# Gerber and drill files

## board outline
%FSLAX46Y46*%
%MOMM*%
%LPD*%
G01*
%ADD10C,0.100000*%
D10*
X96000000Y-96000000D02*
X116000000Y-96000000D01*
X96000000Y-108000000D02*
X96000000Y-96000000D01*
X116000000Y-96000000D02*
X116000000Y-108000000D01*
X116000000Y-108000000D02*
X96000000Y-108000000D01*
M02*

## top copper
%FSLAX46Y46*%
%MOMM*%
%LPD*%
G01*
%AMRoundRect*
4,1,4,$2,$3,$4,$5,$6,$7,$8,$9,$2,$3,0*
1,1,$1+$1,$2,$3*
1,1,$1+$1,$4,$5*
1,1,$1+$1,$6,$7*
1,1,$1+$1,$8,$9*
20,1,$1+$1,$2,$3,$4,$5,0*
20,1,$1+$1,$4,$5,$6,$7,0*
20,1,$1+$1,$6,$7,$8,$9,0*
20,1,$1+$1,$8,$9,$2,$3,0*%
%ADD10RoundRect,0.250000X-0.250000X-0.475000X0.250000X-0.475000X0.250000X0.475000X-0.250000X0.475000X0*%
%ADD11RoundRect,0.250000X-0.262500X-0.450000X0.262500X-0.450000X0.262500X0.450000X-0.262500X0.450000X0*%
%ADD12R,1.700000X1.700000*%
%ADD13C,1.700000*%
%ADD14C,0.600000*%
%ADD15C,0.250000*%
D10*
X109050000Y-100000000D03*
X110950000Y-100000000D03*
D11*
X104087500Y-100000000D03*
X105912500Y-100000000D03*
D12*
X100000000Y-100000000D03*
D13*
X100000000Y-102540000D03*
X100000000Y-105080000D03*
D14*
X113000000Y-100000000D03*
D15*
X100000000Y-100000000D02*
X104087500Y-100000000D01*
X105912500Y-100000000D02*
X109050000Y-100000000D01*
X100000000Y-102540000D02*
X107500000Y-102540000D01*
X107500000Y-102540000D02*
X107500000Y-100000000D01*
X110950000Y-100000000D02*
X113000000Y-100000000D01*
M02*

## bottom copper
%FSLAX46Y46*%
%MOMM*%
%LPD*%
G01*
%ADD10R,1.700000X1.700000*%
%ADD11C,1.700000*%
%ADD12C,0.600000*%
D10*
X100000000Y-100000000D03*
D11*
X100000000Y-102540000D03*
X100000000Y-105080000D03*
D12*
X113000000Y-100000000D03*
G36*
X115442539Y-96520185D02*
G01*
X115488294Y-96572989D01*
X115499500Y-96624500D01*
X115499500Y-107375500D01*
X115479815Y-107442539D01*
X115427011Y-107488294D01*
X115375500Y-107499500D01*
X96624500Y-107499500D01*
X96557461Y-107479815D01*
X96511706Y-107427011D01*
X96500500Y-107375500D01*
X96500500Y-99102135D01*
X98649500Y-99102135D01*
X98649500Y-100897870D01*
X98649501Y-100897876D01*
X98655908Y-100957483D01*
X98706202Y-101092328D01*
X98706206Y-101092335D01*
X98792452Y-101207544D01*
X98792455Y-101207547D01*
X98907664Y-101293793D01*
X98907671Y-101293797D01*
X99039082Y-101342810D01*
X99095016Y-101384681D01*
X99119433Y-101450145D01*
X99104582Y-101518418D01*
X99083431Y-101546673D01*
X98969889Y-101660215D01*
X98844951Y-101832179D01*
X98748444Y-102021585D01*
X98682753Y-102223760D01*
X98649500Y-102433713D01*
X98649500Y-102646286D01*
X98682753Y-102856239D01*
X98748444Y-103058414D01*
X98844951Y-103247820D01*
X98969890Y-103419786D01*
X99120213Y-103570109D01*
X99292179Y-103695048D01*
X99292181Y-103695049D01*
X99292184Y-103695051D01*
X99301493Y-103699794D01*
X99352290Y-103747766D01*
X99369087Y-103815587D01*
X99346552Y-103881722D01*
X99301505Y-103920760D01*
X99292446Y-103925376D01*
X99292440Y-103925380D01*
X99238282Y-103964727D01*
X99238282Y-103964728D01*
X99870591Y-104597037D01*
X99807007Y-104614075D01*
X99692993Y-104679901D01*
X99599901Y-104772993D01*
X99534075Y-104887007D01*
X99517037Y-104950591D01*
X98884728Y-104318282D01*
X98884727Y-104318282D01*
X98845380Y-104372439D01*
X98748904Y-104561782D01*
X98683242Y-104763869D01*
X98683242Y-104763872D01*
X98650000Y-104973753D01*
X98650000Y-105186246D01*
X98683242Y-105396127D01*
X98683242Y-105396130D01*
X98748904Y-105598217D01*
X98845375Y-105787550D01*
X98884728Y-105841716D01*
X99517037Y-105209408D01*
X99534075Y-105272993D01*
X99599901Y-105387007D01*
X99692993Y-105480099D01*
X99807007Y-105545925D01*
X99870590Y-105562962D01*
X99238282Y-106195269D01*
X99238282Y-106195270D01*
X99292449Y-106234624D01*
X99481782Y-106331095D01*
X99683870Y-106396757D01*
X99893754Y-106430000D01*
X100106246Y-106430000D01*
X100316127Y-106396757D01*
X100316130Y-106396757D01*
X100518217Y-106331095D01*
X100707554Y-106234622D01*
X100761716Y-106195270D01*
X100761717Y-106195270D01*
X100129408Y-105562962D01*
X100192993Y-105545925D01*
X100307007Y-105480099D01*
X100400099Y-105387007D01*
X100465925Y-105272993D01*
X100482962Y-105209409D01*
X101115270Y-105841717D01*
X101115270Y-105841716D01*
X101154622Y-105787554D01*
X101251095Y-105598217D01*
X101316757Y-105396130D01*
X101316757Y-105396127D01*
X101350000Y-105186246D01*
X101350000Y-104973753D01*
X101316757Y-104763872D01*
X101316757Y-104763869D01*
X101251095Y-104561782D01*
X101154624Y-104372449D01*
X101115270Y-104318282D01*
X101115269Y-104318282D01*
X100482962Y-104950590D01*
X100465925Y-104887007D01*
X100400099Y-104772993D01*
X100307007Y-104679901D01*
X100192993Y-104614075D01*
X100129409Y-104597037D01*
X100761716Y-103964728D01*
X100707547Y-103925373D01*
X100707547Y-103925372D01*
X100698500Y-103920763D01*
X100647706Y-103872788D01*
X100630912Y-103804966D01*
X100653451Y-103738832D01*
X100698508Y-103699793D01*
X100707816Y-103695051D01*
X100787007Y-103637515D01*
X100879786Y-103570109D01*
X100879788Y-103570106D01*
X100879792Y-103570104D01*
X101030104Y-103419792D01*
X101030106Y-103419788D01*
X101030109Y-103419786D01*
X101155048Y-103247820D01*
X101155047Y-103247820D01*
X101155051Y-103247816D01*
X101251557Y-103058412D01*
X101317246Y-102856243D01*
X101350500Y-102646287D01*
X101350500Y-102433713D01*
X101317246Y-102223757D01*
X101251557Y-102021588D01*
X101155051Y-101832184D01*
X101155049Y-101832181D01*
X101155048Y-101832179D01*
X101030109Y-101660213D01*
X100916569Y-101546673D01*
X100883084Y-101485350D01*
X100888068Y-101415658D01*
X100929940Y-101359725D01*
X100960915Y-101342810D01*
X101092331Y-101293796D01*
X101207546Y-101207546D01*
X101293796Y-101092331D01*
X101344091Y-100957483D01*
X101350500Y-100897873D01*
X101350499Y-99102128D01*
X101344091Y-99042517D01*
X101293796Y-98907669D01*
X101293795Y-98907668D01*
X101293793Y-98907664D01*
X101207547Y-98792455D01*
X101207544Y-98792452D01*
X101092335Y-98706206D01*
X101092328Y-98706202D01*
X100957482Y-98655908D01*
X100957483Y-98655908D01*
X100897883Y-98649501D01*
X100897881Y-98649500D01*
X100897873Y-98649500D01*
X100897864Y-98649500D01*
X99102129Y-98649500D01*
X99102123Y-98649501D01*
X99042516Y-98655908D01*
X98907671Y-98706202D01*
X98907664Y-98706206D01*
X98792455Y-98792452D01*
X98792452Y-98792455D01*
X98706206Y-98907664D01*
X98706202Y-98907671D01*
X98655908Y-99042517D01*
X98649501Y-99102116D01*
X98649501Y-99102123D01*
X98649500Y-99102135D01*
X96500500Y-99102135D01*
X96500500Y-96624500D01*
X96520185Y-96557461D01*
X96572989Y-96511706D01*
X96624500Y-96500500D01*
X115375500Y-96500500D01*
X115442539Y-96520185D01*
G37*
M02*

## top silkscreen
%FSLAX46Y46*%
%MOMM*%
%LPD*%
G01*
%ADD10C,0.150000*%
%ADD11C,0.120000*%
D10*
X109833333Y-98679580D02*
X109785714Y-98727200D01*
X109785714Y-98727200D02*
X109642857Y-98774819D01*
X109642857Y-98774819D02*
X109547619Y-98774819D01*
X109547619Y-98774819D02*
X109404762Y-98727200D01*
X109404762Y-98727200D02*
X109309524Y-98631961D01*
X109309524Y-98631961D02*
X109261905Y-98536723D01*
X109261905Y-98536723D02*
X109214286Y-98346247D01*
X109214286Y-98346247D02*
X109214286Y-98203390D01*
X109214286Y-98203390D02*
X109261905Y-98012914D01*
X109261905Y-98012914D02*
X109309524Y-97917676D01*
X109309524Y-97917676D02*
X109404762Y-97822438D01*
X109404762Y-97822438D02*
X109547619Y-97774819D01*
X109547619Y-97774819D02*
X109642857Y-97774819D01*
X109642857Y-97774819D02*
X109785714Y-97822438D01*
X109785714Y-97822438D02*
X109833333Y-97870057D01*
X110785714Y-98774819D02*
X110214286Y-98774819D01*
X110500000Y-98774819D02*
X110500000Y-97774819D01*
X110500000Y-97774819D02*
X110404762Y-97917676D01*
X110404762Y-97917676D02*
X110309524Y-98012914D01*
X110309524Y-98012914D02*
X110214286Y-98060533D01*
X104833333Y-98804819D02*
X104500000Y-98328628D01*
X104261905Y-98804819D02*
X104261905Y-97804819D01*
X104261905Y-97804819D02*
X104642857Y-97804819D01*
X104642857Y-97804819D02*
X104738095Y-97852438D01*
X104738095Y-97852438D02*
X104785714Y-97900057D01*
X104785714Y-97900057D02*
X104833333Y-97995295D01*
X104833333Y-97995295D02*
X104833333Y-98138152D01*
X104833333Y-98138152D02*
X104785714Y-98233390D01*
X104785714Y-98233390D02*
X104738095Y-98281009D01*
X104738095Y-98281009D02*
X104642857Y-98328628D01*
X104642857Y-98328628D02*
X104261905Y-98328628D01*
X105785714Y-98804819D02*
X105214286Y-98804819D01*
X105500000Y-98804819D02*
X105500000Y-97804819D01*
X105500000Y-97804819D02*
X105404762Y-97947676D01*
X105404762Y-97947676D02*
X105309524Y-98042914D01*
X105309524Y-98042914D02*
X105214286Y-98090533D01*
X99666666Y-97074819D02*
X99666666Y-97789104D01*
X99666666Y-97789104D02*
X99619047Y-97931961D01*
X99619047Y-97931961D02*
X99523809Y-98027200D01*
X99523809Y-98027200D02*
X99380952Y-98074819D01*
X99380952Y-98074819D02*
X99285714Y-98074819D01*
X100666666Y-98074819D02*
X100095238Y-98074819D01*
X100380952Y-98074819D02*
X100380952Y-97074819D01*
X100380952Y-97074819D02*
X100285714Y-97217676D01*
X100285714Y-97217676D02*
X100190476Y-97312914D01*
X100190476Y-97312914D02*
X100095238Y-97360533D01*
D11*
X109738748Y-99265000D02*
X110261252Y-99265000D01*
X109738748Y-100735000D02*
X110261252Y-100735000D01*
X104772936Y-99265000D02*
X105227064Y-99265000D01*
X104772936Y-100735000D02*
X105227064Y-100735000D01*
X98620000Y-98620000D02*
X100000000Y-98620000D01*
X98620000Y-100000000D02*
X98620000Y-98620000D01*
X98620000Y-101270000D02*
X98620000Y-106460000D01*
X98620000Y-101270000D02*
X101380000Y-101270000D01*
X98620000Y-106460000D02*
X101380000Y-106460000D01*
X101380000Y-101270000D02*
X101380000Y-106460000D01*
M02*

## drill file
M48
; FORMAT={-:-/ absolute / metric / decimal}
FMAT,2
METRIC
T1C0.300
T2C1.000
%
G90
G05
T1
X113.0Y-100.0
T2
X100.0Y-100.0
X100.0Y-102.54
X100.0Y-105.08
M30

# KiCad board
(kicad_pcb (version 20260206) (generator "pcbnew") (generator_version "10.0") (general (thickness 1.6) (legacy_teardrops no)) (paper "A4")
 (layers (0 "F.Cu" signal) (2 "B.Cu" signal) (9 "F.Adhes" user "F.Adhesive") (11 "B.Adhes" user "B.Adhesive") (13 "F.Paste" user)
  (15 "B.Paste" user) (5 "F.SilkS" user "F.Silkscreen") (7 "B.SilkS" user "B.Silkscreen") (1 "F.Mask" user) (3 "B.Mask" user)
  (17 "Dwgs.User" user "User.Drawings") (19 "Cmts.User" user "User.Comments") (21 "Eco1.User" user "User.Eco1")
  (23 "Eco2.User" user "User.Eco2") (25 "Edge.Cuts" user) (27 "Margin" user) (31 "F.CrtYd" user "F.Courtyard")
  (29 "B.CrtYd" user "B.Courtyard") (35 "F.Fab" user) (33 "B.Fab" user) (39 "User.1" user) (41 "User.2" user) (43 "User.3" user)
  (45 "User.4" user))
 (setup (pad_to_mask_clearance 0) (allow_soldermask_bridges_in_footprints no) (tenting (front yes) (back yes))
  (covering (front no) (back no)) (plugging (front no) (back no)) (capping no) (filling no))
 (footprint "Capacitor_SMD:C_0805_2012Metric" (layer "F.Cu") (at 110 100)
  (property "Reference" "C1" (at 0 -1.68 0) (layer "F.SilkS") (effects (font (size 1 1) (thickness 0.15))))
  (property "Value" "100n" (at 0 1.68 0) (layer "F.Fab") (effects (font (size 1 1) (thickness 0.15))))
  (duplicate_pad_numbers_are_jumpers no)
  (fp_line (start -0.261252 -0.735) (end 0.261252 -0.735) (stroke (width 0.12) (type solid)) (layer "F.SilkS"))
  (fp_line (start -0.261252 0.735) (end 0.261252 0.735) (stroke (width 0.12) (type solid)) (layer "F.SilkS"))
  (pad "1" smd roundrect (at -0.95 0) (size 1 1.45) (layers "F.Cu" "F.Mask" "F.Paste") (roundrect_rratio 0.25) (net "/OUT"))
  (pad "2" smd roundrect (at 0.95 0) (size 1 1.45) (layers "F.Cu" "F.Mask" "F.Paste") (roundrect_rratio 0.25) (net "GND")))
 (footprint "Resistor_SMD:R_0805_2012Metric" (layer "F.Cu") (at 105 100)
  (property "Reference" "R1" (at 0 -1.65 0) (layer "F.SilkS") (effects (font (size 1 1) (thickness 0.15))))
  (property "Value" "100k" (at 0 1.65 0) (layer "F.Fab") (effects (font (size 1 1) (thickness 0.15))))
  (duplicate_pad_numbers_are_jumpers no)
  (fp_line (start -0.227064 -0.735) (end 0.227064 -0.735) (stroke (width 0.12) (type solid)) (layer "F.SilkS"))
  (fp_line (start -0.227064 0.735) (end 0.227064 0.735) (stroke (width 0.12) (type solid)) (layer "F.SilkS"))
  (pad "1" smd roundrect (at -0.9125 0) (size 1.025 1.4) (layers "F.Cu" "F.Mask" "F.Paste") (roundrect_rratio 0.243902) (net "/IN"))
  (pad "2" smd roundrect (at 0.9125 0) (size 1.025 1.4) (layers "F.Cu" "F.Mask" "F.Paste") (roundrect_rratio 0.243902) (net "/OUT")))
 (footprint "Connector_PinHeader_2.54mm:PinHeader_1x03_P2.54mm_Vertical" (layer "F.Cu") (at 100 100)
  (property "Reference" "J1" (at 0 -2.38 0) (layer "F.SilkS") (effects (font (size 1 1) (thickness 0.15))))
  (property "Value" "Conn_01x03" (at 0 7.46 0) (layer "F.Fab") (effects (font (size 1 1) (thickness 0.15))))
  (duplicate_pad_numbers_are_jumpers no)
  (fp_line (start -1.38 -1.38) (end 0 -1.38) (stroke (width 0.12) (type solid)) (layer "F.SilkS"))
  (fp_line (start -1.38 0) (end -1.38 -1.38) (stroke (width 0.12) (type solid)) (layer "F.SilkS"))
  (fp_line (start -1.38 1.27) (end -1.38 6.46) (stroke (width 0.12) (type solid)) (layer "F.SilkS"))
  (fp_line (start -1.38 1.27) (end 1.38 1.27) (stroke (width 0.12) (type solid)) (layer "F.SilkS"))
  (fp_line (start -1.38 6.46) (end 1.38 6.46) (stroke (width 0.12) (type solid)) (layer "F.SilkS"))
  (fp_line (start 1.38 1.27) (end 1.38 6.46) (stroke (width 0.12) (type solid)) (layer "F.SilkS"))
  (pad "1" thru_hole rect (at 0 0) (size 1.7 1.7) (drill 1) (layers "*.Cu" "*.Mask") (remove_unused_layers no) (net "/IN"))
  (pad "2" thru_hole circle (at 0 2.54) (size 1.7 1.7) (drill 1) (layers "*.Cu" "*.Mask") (remove_unused_layers no) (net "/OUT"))
  (pad "3" thru_hole circle (at 0 5.08) (size 1.7 1.7) (drill 1) (layers "*.Cu" "*.Mask") (remove_unused_layers no) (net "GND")))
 (gr_line (start 96 96) (end 116 96) (stroke (width 0.1) (type default)) (layer "Edge.Cuts"))
 (gr_line (start 96 108) (end 96 96) (stroke (width 0.1) (type default)) (layer "Edge.Cuts"))
 (gr_line (start 116 96) (end 116 108) (stroke (width 0.1) (type default)) (layer "Edge.Cuts"))
 (gr_line (start 116 108) (end 96 108) (stroke (width 0.1) (type default)) (layer "Edge.Cuts"))
 (segment (start 100 100) (end 104.0875 100) (width 0.25) (layer "F.Cu") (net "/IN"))
 (segment (start 105.9125 100) (end 109.05 100) (width 0.25) (layer "F.Cu") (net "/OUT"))
 (segment (start 100 102.54) (end 107.5 102.54) (width 0.25) (layer "F.Cu") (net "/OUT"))
 (segment (start 107.5 102.54) (end 107.5 100) (width 0.25) (layer "F.Cu") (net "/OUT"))
 (segment (start 110.95 100) (end 113 100) (width 0.25) (layer "F.Cu") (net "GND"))
 (via (at 113 100) (size 0.6) (drill 0.3) (layers "F.Cu" "B.Cu") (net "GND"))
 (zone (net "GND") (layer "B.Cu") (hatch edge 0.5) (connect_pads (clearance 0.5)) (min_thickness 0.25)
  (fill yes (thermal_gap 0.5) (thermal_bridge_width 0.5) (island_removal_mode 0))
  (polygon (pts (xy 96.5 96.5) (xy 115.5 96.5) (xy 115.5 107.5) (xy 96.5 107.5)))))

